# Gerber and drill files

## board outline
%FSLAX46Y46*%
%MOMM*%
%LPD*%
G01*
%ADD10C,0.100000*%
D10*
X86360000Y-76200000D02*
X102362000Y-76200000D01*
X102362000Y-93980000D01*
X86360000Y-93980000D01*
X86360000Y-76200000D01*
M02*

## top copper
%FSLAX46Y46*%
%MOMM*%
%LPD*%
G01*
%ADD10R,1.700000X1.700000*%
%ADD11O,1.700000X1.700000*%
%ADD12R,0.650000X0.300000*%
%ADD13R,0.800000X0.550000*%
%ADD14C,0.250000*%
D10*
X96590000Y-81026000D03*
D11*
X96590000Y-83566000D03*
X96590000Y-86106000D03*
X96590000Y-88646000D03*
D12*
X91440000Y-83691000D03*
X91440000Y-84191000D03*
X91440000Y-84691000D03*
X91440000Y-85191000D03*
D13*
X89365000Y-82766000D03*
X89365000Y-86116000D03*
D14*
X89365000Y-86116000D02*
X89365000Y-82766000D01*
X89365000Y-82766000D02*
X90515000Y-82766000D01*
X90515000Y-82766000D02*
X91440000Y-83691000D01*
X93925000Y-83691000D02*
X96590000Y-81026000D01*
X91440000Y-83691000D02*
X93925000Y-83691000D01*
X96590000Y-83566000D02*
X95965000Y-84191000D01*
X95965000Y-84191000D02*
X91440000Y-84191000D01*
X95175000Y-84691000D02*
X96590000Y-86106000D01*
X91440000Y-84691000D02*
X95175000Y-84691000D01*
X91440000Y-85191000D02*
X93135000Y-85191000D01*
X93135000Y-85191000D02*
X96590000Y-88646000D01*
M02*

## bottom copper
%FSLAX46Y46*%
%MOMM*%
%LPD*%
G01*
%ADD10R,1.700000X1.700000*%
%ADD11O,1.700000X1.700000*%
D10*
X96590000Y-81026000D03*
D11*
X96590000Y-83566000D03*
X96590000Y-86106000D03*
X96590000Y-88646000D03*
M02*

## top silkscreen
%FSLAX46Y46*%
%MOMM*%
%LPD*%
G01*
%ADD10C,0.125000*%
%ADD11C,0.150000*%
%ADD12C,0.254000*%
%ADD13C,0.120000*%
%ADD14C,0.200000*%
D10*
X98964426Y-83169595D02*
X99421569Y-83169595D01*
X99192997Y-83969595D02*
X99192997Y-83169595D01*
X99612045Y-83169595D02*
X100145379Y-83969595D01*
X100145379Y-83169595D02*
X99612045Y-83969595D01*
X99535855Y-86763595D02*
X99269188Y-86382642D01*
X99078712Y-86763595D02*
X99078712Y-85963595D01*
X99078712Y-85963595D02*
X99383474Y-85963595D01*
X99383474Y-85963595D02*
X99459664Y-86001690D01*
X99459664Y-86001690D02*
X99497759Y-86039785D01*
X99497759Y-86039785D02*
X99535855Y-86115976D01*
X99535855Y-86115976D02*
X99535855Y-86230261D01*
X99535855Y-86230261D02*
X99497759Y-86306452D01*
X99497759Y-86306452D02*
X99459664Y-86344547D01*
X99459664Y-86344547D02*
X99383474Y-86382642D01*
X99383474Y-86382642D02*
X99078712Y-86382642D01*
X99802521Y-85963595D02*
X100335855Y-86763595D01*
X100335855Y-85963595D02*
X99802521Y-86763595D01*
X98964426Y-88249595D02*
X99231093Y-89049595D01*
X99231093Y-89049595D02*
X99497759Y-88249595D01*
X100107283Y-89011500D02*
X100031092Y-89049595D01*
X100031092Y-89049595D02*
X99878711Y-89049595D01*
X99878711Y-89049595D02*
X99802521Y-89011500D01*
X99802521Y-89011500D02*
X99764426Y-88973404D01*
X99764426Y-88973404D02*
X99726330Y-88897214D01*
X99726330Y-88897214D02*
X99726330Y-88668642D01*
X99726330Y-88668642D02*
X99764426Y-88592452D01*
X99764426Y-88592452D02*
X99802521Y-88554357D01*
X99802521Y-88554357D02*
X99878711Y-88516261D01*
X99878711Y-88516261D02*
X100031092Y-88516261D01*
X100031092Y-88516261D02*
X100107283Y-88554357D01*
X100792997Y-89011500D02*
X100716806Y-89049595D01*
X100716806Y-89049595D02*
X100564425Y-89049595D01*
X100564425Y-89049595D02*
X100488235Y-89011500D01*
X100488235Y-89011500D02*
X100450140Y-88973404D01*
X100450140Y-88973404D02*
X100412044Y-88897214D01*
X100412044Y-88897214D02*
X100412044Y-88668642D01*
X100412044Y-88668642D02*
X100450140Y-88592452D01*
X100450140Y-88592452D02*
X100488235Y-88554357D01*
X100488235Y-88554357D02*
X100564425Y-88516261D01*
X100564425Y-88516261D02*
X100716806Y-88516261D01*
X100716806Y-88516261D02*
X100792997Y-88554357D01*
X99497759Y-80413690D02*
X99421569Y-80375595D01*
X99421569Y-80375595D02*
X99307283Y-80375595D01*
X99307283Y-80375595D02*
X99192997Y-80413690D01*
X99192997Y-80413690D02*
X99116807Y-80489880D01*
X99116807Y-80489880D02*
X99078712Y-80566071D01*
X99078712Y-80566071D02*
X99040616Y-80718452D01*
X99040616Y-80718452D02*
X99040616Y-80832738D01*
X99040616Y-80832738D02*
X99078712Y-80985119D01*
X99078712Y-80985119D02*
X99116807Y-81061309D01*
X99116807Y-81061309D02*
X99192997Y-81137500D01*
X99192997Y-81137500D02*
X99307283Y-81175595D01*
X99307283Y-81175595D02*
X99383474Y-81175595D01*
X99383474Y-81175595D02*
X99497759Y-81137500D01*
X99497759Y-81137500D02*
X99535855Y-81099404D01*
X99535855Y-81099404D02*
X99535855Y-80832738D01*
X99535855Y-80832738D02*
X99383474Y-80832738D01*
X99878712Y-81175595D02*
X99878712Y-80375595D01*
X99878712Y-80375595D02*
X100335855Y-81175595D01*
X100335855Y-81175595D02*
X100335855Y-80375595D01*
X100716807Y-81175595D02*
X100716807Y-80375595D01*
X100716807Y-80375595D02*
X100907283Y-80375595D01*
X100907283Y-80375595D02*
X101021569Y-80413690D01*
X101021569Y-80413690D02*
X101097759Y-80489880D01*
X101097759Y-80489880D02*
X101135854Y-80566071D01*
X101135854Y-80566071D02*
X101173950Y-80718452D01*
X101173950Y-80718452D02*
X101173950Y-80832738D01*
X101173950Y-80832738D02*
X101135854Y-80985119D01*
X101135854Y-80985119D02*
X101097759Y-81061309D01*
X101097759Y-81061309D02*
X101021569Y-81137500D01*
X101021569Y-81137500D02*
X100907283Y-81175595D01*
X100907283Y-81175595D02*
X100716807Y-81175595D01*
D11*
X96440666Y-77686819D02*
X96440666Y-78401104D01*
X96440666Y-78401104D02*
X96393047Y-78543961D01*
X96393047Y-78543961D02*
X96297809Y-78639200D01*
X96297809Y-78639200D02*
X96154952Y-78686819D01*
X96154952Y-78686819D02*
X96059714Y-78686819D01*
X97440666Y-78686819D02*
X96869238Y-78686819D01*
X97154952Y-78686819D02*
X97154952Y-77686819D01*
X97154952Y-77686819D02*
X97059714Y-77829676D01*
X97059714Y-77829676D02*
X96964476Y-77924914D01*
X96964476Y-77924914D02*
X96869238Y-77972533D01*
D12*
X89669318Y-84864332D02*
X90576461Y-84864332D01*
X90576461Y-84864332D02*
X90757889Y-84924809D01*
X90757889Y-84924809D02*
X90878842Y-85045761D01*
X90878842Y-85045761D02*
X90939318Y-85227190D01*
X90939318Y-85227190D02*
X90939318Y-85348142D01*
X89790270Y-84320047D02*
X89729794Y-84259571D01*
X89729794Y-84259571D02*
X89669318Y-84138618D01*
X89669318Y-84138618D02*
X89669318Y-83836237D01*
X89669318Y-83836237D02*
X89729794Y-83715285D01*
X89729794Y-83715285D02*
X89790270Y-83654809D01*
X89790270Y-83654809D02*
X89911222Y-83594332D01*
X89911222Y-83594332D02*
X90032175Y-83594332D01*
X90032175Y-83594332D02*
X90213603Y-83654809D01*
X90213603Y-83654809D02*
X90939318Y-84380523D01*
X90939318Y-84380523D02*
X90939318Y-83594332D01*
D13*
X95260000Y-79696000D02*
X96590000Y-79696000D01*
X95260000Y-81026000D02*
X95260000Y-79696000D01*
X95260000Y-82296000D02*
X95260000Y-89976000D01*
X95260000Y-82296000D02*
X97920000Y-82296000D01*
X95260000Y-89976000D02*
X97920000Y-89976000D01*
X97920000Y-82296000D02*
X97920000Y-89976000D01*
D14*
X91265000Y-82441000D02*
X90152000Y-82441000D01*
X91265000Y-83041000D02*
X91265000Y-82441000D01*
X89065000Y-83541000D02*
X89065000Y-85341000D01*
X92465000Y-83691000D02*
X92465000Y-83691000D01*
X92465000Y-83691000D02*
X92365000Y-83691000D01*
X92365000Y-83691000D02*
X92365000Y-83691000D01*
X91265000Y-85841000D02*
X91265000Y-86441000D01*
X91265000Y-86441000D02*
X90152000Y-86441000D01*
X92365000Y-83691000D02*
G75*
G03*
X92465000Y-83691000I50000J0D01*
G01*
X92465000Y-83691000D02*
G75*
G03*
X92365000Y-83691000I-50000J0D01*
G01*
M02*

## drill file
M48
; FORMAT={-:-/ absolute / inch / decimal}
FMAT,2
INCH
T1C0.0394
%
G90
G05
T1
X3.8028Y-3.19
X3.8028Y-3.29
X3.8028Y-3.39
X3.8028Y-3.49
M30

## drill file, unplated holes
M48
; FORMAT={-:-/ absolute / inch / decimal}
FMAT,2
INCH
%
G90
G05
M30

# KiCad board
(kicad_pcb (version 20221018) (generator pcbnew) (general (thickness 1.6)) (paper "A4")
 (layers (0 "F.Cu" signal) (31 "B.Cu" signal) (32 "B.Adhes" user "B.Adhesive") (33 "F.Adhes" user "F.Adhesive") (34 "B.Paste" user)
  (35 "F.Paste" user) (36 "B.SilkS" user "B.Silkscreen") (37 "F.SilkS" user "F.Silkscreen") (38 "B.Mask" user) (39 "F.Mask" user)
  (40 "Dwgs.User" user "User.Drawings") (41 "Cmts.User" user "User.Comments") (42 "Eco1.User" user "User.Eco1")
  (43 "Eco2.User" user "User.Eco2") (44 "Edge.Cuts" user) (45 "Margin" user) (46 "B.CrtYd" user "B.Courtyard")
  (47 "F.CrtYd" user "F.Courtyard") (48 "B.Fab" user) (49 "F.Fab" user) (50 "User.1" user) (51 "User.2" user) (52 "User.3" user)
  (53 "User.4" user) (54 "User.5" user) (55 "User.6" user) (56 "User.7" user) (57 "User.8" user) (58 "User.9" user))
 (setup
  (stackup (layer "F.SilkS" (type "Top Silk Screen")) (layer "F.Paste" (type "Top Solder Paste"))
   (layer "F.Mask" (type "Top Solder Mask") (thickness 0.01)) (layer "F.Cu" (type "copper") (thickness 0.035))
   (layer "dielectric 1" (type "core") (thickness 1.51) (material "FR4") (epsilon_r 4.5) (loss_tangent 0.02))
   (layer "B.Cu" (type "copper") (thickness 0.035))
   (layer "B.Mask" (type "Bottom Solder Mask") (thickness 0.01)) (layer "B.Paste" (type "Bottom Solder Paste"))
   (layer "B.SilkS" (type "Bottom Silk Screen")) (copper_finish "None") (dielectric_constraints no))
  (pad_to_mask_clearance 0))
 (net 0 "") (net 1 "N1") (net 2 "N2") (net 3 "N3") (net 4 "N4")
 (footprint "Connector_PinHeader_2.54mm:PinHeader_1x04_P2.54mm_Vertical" (layer "F.Cu") (at 96.59 81.026)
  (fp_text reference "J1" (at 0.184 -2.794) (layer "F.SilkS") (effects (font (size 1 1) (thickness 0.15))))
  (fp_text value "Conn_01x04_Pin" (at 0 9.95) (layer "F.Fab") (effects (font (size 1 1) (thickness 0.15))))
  (fp_line (start -1.33 -1.33) (end 0 -1.33) (stroke (width 0.12) (type solid)) (layer "F.SilkS"))
  (fp_line (start -1.33 0) (end -1.33 -1.33) (stroke (width 0.12) (type solid)) (layer "F.SilkS"))
  (fp_line (start -1.33 1.27) (end -1.33 8.95) (stroke (width 0.12) (type solid)) (layer "F.SilkS"))
  (fp_line (start -1.33 1.27) (end 1.33 1.27) (stroke (width 0.12) (type solid)) (layer "F.SilkS"))
  (fp_line (start -1.33 8.95) (end 1.33 8.95) (stroke (width 0.12) (type solid)) (layer "F.SilkS"))
  (fp_line (start 1.33 1.27) (end 1.33 8.95) (stroke (width 0.12) (type solid)) (layer "F.SilkS"))
  (pad "1" thru_hole rect (at 0 0) (size 1.7 1.7) (drill 1) (layers "*.Cu" "*.Mask") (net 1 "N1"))
  (pad "2" thru_hole oval (at 0 2.54) (size 1.7 1.7) (drill 1) (layers "*.Cu" "*.Mask") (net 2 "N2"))
  (pad "3" thru_hole oval (at 0 5.08) (size 1.7 1.7) (drill 1) (layers "*.Cu" "*.Mask") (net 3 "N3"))
  (pad "4" thru_hole oval (at 0 7.62) (size 1.7 1.7) (drill 1) (layers "*.Cu" "*.Mask") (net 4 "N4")))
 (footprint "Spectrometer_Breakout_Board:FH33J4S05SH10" (layer "F.Cu") (at 90.165 84.441 -90)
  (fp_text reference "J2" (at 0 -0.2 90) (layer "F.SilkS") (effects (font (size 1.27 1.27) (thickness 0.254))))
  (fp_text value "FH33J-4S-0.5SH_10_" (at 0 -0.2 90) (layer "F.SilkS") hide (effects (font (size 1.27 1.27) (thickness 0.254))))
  (fp_line (start -2 -1.1) (end -2 0.013) (stroke (width 0.2) (type solid)) (layer "F.SilkS"))
  (fp_line (start -1.4 -1.1) (end -2 -1.1) (stroke (width 0.2) (type solid)) (layer "F.SilkS"))
  (fp_line (start -0.9 1.1) (end 0.9 1.1) (stroke (width 0.2) (type solid)) (layer "F.SilkS"))
  (fp_line (start -0.75 -2.3) (end -0.75 -2.3) (stroke (width 0.2) (type solid)) (layer "F.SilkS"))
  (fp_line (start -0.75 -2.3) (end -0.75 -2.2) (stroke (width 0.2) (type solid)) (layer "F.SilkS"))
  (fp_line (start -0.75 -2.2) (end -0.75 -2.2) (stroke (width 0.2) (type solid)) (layer "F.SilkS"))
  (fp_line (start 1.4 -1.1) (end 2 -1.1) (stroke (width 0.2) (type solid)) (layer "F.SilkS"))
  (fp_line (start 2 -1.1) (end 2 0.013) (stroke (width 0.2) (type solid)) (layer "F.SilkS"))
  (fp_arc (start -0.75 -2.3) (mid -0.7 -2.25) (end -0.75 -2.2) (stroke (width 0.2) (type solid)) (layer "F.SilkS"))
  (fp_arc (start -0.75 -2.2) (mid -0.8 -2.25) (end -0.75 -2.3) (stroke (width 0.2) (type solid)) (layer "F.SilkS"))
  (pad "1" smd rect (at -0.75 -1.275 270) (size 0.3 0.65) (layers "F.Cu" "F.Paste" "F.Mask") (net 1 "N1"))
  (pad "2" smd rect (at -0.25 -1.275 270) (size 0.3 0.65) (layers "F.Cu" "F.Paste" "F.Mask") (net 2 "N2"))
  (pad "3" smd rect (at 0.25 -1.275 270) (size 0.3 0.65) (layers "F.Cu" "F.Paste" "F.Mask") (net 3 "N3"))
  (pad "4" smd rect (at 0.75 -1.275 270) (size 0.3 0.65) (layers "F.Cu" "F.Paste" "F.Mask") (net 4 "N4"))
  (pad "MP1" smd rect (at -1.675 0.8 270) (size 0.55 0.8) (layers "F.Cu" "F.Paste" "F.Mask") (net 1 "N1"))
  (pad "MP2" smd rect (at 1.675 0.8 270) (size 0.55 0.8) (layers "F.Cu" "F.Paste" "F.Mask") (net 1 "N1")))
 (gr_rect (start 86.36 76.2) (end 102.362 93.98) (stroke (width 0.1) (type default)) (fill none) (layer "Edge.Cuts"))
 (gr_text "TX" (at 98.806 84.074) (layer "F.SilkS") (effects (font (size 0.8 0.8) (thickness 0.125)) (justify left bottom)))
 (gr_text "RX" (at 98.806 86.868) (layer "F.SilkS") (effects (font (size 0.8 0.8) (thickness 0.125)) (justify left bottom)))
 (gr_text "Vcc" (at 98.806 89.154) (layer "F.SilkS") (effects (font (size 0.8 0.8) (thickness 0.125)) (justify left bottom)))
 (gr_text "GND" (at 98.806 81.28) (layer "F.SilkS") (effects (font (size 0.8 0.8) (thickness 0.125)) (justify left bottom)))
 (segment (start 89.365 86.116) (end 89.365 82.766) (width 0.25) (layer "F.Cu") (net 1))
 (segment (start 89.365 82.766) (end 90.515 82.766) (width 0.25) (layer "F.Cu") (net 1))
 (segment (start 90.515 82.766) (end 91.44 83.691) (width 0.25) (layer "F.Cu") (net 1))
 (segment (start 93.925 83.691) (end 96.59 81.026) (width 0.25) (layer "F.Cu") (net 1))
 (segment (start 91.44 83.691) (end 93.925 83.691) (width 0.25) (layer "F.Cu") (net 1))
 (segment (start 96.59 83.566) (end 95.965 84.191) (width 0.25) (layer "F.Cu") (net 2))
 (segment (start 95.965 84.191) (end 91.44 84.191) (width 0.25) (layer "F.Cu") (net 2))
 (segment (start 95.175 84.691) (end 96.59 86.106) (width 0.25) (layer "F.Cu") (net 3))
 (segment (start 91.44 84.691) (end 95.175 84.691) (width 0.25) (layer "F.Cu") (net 3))
 (segment (start 91.44 85.191) (end 93.135 85.191) (width 0.25) (layer "F.Cu") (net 4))
 (segment (start 93.135 85.191) (end 96.59 88.646) (width 0.25) (layer "F.Cu") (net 4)))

